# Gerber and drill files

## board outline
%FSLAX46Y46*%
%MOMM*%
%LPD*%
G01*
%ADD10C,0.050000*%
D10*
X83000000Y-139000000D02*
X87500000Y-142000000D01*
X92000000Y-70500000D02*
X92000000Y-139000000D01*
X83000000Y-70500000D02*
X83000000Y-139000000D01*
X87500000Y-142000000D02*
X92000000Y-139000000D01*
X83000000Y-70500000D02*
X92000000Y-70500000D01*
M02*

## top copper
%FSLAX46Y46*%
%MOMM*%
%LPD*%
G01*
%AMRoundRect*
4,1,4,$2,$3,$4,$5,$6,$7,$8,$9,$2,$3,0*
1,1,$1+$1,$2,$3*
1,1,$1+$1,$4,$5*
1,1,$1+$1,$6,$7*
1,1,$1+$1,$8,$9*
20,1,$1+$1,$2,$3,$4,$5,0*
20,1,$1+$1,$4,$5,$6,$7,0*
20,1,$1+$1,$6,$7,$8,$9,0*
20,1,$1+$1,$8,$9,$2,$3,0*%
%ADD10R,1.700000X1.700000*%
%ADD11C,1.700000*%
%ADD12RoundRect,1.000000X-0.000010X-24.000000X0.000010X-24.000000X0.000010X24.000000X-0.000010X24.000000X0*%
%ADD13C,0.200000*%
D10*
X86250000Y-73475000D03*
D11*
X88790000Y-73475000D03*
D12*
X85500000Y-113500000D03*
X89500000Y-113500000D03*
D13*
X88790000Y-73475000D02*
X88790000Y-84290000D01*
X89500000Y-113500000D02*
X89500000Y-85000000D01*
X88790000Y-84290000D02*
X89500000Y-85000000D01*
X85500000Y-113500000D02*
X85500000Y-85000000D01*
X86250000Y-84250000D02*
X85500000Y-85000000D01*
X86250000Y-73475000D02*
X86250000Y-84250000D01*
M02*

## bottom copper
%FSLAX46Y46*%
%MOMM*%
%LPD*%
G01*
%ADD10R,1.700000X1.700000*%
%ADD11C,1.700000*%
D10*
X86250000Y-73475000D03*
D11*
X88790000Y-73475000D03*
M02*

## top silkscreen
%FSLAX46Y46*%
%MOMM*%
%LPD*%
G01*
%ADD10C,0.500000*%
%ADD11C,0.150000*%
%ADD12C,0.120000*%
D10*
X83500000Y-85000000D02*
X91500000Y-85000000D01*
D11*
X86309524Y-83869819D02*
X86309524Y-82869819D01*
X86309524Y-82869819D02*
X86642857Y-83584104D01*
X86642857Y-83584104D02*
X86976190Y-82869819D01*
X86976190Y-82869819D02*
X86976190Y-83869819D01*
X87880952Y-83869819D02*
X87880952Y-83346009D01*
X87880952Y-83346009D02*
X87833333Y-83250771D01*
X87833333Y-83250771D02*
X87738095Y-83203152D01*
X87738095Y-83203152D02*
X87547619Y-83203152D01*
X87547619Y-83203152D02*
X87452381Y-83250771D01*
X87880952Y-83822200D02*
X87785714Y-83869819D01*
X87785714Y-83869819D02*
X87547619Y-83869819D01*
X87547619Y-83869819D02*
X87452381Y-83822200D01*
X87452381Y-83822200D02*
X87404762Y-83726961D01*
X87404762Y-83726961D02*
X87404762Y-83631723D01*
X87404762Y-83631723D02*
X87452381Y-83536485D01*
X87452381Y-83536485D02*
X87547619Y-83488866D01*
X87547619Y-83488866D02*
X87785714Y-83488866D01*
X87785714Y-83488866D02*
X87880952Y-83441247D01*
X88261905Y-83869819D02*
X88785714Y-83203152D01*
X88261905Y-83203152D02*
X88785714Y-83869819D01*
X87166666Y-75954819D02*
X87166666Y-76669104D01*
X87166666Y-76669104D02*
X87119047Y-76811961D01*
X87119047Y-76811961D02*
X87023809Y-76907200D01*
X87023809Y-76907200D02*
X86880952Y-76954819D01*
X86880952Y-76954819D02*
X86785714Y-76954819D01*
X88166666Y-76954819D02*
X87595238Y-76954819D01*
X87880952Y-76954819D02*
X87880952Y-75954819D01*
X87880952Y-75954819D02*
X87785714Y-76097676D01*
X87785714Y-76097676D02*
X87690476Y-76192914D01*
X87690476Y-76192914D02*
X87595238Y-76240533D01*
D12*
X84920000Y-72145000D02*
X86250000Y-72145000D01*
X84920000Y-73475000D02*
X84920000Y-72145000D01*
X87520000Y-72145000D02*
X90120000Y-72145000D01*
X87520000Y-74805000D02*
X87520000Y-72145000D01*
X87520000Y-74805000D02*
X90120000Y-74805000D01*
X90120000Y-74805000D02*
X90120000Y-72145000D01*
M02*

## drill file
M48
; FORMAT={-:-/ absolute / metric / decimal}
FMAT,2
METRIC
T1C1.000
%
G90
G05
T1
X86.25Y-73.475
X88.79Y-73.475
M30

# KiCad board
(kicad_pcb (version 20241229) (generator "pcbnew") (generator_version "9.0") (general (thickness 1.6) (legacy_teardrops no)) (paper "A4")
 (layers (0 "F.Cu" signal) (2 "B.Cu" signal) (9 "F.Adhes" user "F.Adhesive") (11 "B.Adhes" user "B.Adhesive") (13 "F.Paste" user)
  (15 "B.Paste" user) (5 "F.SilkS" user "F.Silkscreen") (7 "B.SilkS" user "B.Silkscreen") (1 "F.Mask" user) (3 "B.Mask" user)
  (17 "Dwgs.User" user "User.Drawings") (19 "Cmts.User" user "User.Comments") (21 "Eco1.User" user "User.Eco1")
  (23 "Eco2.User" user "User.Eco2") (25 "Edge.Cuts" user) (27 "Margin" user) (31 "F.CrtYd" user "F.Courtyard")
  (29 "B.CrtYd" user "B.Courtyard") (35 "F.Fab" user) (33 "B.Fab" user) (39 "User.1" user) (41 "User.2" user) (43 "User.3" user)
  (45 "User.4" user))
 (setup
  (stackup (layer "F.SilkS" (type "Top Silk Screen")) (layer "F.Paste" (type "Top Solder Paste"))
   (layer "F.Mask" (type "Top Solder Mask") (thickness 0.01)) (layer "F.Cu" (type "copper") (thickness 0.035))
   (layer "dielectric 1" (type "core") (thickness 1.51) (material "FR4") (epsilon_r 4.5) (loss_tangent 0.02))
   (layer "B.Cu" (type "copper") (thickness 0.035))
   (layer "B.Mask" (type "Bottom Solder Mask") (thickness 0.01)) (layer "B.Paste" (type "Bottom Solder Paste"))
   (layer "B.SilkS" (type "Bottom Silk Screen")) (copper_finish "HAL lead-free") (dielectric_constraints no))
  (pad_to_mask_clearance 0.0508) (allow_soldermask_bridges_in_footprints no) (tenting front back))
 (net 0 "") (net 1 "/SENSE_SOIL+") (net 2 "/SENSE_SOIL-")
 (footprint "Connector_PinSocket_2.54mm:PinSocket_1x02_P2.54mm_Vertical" (layer "F.Cu") (at 86.25 73.475 90)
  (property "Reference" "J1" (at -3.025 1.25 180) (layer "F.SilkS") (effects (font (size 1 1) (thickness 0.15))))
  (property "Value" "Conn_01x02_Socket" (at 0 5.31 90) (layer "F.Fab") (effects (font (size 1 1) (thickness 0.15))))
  (fp_line (start 1.33 -1.33) (end 1.33 0) (stroke (width 0.12) (type solid)) (layer "F.SilkS"))
  (fp_line (start 0 -1.33) (end 1.33 -1.33) (stroke (width 0.12) (type solid)) (layer "F.SilkS"))
  (fp_line (start 1.33 1.27) (end 1.33 3.87) (stroke (width 0.12) (type solid)) (layer "F.SilkS"))
  (fp_line (start -1.33 1.27) (end 1.33 1.27) (stroke (width 0.12) (type solid)) (layer "F.SilkS"))
  (fp_line (start -1.33 1.27) (end -1.33 3.87) (stroke (width 0.12) (type solid)) (layer "F.SilkS"))
  (fp_line (start -1.33 3.87) (end 1.33 3.87) (stroke (width 0.12) (type solid)) (layer "F.SilkS"))
  (pad "1" thru_hole rect (at 0 0 90) (size 1.7 1.7) (drill 1) (layers "*.Cu" "*.Mask") (remove_unused_layers no) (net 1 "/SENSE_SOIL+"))
  (pad "2" thru_hole circle (at 0 2.54 90) (size 1.7 1.7) (drill 1) (layers "*.Cu" "*.Mask") (remove_unused_layers no)
   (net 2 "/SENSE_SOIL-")))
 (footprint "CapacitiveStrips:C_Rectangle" (layer "F.Cu") (at 87.5 88.5)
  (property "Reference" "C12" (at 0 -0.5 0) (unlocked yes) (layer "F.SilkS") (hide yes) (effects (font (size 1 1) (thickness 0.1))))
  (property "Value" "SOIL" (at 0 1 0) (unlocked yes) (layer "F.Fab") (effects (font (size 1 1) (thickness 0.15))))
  (pad "1" smd roundrect (at -2 25) (size 2 50) (layers "F.Cu") (roundrect_rratio 0.5) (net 1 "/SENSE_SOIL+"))
  (pad "2" smd roundrect (at 2 25) (size 2 50) (layers "F.Cu") (roundrect_rratio 0.5) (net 2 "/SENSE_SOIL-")))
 (gr_line (start 83.5 85) (end 91.5 85) (stroke (width 0.5) (type solid)) (layer "F.SilkS"))
 (gr_line (start 83 139) (end 87.5 142) (stroke (width 0.05) (type default)) (layer "Edge.Cuts"))
 (gr_line (start 92 70.5) (end 92 139) (stroke (width 0.05) (type default)) (layer "Edge.Cuts"))
 (gr_line (start 83 70.5) (end 83 139) (stroke (width 0.05) (type default)) (layer "Edge.Cuts"))
 (gr_line (start 87.5 142) (end 92 139) (stroke (width 0.05) (type default)) (layer "Edge.Cuts"))
 (gr_line (start 83 70.5) (end 92 70.5) (stroke (width 0.05) (type default)) (layer "Edge.Cuts"))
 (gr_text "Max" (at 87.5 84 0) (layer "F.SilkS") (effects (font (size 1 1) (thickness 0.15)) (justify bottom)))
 (segment (start 88.79 73.475) (end 88.79 84.29) (width 0.2) (layer "F.Cu") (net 2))
 (segment (start 89.5 113.5) (end 89.5 85) (width 0.2) (layer "F.Cu") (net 2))
 (segment (start 88.79 84.29) (end 89.5 85) (width 0.2) (layer "F.Cu") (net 2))
 (segment (start 85.5 113.5) (end 85.5 85) (width 0.2) (layer "F.Cu") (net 1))
 (segment (start 86.25 84.25) (end 85.5 85) (width 0.2) (layer "F.Cu") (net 1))
 (segment (start 86.25 73.475) (end 86.25 84.25) (width 0.2) (layer "F.Cu") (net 1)))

